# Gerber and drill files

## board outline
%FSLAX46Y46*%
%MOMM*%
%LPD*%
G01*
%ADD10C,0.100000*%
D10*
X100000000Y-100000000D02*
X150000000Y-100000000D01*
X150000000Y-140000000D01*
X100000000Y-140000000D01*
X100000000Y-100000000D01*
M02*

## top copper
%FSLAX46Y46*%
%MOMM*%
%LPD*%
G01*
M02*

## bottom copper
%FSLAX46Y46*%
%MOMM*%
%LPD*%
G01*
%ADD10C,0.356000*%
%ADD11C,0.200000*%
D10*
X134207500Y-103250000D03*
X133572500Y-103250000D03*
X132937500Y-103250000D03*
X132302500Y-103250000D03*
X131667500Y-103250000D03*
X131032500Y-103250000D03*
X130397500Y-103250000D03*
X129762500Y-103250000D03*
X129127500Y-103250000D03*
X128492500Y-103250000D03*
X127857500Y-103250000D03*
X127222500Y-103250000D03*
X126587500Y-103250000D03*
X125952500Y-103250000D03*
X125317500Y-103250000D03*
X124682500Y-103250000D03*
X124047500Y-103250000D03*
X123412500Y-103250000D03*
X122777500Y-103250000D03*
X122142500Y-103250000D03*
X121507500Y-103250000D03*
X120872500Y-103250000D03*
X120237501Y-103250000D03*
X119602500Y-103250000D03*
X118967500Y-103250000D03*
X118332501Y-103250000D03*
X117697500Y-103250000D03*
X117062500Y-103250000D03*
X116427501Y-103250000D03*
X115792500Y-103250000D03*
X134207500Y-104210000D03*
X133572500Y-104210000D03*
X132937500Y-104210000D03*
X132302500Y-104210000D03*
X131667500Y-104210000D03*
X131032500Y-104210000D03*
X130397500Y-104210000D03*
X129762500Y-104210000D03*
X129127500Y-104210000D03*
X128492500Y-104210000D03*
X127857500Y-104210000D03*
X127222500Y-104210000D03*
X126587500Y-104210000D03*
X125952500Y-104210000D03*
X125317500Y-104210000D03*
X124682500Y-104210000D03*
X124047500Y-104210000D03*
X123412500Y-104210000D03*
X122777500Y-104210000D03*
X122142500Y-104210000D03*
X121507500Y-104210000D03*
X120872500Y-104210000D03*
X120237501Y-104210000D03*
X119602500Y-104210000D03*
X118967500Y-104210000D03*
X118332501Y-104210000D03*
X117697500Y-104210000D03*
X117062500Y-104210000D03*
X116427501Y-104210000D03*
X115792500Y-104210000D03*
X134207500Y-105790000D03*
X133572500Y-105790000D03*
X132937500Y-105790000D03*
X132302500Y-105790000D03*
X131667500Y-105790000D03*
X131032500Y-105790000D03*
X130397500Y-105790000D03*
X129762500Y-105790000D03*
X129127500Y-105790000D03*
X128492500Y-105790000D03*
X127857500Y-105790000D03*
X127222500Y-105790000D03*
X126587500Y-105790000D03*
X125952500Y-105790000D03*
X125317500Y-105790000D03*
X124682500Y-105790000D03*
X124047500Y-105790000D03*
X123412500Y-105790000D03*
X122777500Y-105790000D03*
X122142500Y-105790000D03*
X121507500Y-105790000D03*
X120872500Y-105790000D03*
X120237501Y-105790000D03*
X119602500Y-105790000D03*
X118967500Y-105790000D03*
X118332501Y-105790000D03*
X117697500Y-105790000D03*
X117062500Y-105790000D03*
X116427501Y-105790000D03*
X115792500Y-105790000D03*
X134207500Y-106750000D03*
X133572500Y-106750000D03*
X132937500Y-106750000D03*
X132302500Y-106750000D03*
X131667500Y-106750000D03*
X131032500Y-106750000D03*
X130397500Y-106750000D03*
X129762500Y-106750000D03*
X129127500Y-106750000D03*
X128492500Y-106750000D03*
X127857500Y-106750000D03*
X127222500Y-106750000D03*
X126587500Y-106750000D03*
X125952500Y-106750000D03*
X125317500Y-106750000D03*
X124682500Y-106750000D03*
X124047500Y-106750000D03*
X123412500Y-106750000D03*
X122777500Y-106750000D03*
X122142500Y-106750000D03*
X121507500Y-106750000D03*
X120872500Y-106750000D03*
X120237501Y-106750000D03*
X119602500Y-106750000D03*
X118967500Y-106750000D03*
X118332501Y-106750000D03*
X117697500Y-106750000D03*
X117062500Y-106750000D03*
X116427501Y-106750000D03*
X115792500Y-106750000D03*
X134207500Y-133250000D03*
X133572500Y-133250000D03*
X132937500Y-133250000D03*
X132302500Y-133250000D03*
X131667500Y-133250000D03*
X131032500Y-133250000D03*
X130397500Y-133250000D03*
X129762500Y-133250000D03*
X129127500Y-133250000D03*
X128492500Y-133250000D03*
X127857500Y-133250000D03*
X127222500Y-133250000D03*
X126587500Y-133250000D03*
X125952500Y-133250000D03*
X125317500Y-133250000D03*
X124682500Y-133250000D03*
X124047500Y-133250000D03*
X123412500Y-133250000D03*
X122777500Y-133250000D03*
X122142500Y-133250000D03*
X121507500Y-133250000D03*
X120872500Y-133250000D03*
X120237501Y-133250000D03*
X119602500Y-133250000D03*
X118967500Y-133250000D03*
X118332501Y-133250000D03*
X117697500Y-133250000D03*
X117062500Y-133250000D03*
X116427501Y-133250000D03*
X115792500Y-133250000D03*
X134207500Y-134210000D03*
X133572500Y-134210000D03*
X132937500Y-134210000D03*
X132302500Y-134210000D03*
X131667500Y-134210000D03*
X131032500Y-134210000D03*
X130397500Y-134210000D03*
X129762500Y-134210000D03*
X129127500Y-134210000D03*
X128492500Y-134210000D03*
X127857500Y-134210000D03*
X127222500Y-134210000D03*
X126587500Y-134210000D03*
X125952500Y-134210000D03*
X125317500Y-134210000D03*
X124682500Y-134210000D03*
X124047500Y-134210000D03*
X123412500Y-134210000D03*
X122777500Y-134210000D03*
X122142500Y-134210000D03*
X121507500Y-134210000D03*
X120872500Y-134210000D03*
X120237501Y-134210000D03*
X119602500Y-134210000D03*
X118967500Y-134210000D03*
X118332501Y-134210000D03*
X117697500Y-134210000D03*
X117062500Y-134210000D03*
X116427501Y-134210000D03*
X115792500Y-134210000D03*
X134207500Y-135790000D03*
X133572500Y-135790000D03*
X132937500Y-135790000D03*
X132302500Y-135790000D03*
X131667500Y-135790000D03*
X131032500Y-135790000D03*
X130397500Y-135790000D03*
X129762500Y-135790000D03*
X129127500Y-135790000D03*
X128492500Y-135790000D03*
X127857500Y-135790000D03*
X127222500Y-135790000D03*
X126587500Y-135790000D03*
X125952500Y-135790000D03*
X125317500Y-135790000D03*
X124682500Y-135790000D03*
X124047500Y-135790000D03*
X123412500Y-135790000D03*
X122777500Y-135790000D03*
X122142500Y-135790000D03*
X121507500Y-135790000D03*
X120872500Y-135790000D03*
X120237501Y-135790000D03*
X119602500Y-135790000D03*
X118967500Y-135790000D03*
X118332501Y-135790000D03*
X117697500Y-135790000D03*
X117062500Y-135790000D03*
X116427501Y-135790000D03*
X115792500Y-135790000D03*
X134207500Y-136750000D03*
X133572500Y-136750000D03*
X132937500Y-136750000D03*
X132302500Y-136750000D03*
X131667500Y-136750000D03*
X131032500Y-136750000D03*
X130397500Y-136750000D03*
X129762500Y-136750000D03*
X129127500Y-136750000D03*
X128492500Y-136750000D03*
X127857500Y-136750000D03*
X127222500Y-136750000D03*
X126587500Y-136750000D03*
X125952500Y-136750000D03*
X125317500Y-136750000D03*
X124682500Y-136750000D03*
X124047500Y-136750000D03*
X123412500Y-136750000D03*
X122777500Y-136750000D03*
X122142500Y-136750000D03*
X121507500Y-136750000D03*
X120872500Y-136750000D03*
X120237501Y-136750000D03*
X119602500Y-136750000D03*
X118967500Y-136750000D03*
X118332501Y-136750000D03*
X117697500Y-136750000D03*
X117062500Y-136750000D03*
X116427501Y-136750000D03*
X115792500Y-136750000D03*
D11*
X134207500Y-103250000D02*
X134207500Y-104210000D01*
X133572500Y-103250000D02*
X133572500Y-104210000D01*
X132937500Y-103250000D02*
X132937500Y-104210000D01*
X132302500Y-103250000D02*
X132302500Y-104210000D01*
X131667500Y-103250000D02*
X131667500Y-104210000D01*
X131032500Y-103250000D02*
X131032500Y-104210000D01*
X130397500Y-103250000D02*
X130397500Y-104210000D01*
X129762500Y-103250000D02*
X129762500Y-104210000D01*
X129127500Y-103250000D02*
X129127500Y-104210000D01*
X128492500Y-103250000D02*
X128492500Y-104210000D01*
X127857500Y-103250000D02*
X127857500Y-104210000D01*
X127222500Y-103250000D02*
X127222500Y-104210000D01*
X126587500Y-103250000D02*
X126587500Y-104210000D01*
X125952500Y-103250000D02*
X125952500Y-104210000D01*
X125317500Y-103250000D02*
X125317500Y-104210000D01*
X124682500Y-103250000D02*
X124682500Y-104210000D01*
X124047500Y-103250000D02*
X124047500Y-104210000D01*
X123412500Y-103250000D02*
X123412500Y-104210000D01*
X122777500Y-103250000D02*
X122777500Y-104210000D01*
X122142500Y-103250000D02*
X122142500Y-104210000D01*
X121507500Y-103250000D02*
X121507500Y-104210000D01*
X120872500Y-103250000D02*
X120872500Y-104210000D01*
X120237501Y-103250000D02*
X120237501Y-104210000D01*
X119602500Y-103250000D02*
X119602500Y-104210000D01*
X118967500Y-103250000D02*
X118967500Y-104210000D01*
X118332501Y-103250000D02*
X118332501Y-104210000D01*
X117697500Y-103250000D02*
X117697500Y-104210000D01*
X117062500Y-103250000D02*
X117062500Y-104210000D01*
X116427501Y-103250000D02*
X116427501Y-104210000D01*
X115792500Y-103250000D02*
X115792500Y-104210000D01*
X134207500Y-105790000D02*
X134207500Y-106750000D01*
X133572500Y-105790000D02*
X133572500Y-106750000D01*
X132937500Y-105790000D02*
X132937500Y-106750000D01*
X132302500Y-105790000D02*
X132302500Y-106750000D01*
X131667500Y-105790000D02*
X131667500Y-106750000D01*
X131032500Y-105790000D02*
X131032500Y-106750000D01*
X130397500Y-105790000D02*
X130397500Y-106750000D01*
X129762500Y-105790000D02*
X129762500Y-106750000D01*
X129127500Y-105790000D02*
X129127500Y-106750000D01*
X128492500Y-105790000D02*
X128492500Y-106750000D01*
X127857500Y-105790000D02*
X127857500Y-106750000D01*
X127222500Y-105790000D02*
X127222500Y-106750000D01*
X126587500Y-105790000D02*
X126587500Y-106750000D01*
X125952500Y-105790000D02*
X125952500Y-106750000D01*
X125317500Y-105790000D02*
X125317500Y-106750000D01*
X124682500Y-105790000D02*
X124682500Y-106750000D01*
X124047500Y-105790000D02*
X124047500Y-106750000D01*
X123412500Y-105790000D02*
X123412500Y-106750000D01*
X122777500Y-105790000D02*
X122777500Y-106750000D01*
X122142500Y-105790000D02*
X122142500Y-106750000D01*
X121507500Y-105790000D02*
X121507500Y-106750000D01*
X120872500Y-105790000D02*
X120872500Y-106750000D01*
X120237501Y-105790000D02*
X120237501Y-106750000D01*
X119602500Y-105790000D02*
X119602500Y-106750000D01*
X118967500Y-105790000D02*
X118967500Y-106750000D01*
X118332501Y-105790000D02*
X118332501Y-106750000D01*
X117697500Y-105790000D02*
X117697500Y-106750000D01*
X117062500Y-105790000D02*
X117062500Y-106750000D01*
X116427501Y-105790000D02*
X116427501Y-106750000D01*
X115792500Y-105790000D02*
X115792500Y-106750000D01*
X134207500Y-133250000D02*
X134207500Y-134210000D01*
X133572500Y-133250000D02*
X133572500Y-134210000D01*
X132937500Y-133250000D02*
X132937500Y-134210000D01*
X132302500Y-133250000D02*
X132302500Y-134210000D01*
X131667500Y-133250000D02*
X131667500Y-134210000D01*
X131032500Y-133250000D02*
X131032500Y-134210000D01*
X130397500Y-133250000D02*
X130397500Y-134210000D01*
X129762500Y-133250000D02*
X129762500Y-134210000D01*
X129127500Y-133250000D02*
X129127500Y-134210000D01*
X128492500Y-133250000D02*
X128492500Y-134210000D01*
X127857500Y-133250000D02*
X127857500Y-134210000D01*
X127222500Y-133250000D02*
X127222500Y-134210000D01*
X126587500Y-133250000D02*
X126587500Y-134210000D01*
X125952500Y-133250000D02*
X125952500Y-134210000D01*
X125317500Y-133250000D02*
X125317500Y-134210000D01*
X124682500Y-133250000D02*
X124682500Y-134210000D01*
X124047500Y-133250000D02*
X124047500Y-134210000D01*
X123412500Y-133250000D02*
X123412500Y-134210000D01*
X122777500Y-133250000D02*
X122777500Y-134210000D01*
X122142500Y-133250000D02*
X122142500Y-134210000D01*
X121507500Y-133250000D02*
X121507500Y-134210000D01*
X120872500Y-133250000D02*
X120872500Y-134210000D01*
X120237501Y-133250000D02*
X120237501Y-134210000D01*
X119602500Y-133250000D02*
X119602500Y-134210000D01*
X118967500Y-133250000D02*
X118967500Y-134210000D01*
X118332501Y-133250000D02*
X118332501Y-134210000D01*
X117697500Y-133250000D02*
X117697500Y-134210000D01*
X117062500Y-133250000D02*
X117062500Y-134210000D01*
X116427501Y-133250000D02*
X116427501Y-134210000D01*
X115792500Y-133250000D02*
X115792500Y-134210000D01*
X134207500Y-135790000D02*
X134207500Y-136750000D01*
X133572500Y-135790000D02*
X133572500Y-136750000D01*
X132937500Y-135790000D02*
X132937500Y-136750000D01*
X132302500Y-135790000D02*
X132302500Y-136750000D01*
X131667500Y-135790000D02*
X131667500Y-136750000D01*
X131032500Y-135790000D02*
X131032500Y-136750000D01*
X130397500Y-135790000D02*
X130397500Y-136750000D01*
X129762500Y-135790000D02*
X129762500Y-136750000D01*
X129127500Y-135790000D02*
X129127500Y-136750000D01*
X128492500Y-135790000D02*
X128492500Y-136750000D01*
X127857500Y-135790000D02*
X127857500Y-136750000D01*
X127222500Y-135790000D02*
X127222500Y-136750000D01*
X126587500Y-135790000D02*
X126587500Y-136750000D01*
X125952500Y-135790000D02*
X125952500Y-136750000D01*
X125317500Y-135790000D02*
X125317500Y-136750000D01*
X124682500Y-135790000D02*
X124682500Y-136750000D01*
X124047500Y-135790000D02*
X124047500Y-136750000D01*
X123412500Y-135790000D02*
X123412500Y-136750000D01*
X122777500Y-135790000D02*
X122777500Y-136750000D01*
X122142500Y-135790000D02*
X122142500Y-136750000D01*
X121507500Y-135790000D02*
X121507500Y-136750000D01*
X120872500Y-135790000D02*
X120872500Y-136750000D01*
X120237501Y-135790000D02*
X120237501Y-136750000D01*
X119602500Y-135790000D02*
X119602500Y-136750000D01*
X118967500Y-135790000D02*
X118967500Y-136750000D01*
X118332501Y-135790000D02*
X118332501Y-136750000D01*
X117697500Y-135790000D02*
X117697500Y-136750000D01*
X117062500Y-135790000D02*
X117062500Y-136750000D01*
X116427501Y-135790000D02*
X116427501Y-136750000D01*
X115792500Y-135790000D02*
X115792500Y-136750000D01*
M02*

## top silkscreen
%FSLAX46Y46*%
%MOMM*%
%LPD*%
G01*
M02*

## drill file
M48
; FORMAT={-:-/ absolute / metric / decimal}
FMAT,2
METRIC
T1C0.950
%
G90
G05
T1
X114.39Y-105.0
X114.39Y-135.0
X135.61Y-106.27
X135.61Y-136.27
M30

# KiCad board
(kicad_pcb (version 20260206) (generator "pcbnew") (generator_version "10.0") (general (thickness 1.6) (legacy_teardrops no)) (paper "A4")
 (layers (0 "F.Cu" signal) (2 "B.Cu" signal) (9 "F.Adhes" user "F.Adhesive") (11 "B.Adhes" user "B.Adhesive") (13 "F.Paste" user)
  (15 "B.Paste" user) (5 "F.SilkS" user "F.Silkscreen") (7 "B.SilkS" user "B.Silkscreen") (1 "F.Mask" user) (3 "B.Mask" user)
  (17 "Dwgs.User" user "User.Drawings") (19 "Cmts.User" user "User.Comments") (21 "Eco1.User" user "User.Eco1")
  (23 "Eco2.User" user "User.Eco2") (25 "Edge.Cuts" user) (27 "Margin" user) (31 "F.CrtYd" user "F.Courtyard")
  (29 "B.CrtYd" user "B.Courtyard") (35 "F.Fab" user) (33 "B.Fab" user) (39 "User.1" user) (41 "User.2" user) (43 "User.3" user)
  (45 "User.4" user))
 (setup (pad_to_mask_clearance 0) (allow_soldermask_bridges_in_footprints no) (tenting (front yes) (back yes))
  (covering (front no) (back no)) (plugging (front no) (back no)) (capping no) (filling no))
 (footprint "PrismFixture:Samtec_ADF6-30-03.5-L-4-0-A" (layer "B.Cu") (at 125 105)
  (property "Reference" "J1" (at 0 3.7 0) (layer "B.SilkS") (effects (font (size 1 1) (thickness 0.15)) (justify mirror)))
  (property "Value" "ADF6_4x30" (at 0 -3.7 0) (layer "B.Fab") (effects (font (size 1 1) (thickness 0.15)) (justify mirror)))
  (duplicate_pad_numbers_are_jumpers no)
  (pad "" np_thru_hole circle (at -10.61 0) (size 0.95 0.95) (drill 0.95) (layers "*.Cu" "*.Mask"))
  (pad "" np_thru_hole circle (at 10.61 1.27) (size 0.95 0.95) (drill 0.95) (layers "*.Cu" "*.Mask"))
  (pad "A01" smd circle (at 9.2075 -1.75) (size 0.356 0.356) (layers "B.Cu" "B.Mask" "B.Paste") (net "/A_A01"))
  (pad "A02" smd circle (at 8.5725 -1.75) (size 0.356 0.356) (layers "B.Cu" "B.Mask" "B.Paste") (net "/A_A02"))
  (pad "A03" smd circle (at 7.9375 -1.75) (size 0.356 0.356) (layers "B.Cu" "B.Mask" "B.Paste") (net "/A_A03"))
  (pad "A04" smd circle (at 7.3025 -1.75) (size 0.356 0.356) (layers "B.Cu" "B.Mask" "B.Paste") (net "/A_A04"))
  (pad "A05" smd circle (at 6.6675 -1.75) (size 0.356 0.356) (layers "B.Cu" "B.Mask" "B.Paste") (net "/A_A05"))
  (pad "A06" smd circle (at 6.0325 -1.75) (size 0.356 0.356) (layers "B.Cu" "B.Mask" "B.Paste") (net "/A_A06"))
  (pad "A07" smd circle (at 5.3975 -1.75) (size 0.356 0.356) (layers "B.Cu" "B.Mask" "B.Paste") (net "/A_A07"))
  (pad "A08" smd circle (at 4.7625 -1.75) (size 0.356 0.356) (layers "B.Cu" "B.Mask" "B.Paste") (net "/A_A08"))
  (pad "A09" smd circle (at 4.1275 -1.75) (size 0.356 0.356) (layers "B.Cu" "B.Mask" "B.Paste") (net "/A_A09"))
  (pad "A10" smd circle (at 3.4925 -1.75) (size 0.356 0.356) (layers "B.Cu" "B.Mask" "B.Paste") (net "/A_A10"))
  (pad "A11" smd circle (at 2.8575 -1.75) (size 0.356 0.356) (layers "B.Cu" "B.Mask" "B.Paste") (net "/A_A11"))
  (pad "A12" smd circle (at 2.2225 -1.75) (size 0.356 0.356) (layers "B.Cu" "B.Mask" "B.Paste") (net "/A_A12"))
  (pad "A13" smd circle (at 1.5875 -1.75) (size 0.356 0.356) (layers "B.Cu" "B.Mask" "B.Paste") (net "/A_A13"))
  (pad "A14" smd circle (at 0.9525 -1.75) (size 0.356 0.356) (layers "B.Cu" "B.Mask" "B.Paste") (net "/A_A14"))
  (pad "A15" smd circle (at 0.3175 -1.75) (size 0.356 0.356) (layers "B.Cu" "B.Mask" "B.Paste") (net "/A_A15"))
  (pad "A16" smd circle (at -0.3175 -1.75) (size 0.356 0.356) (layers "B.Cu" "B.Mask" "B.Paste") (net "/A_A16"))
  (pad "A17" smd circle (at -0.9525 -1.75) (size 0.356 0.356) (layers "B.Cu" "B.Mask" "B.Paste") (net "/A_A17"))
  (pad "A18" smd circle (at -1.5875 -1.75) (size 0.356 0.356) (layers "B.Cu" "B.Mask" "B.Paste") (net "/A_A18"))
  (pad "A19" smd circle (at -2.2225 -1.75) (size 0.356 0.356) (layers "B.Cu" "B.Mask" "B.Paste") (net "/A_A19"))
  (pad "A20" smd circle (at -2.8575 -1.75) (size 0.356 0.356) (layers "B.Cu" "B.Mask" "B.Paste") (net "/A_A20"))
  (pad "A21" smd circle (at -3.4925 -1.75) (size 0.356 0.356) (layers "B.Cu" "B.Mask" "B.Paste") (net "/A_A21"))
  (pad "A22" smd circle (at -4.1275 -1.75) (size 0.356 0.356) (layers "B.Cu" "B.Mask" "B.Paste") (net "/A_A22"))
  (pad "A23" smd circle (at -4.762499 -1.75) (size 0.356 0.356) (layers "B.Cu" "B.Mask" "B.Paste") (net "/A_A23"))
  (pad "A24" smd circle (at -5.3975 -1.75) (size 0.356 0.356) (layers "B.Cu" "B.Mask" "B.Paste") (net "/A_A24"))
  (pad "A25" smd circle (at -6.0325 -1.75) (size 0.356 0.356) (layers "B.Cu" "B.Mask" "B.Paste") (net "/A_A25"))
  (pad "A26" smd circle (at -6.667499 -1.75) (size 0.356 0.356) (layers "B.Cu" "B.Mask" "B.Paste") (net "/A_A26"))
  (pad "A27" smd circle (at -7.3025 -1.75) (size 0.356 0.356) (layers "B.Cu" "B.Mask" "B.Paste") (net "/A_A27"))
  (pad "A28" smd circle (at -7.9375 -1.75) (size 0.356 0.356) (layers "B.Cu" "B.Mask" "B.Paste") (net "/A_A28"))
  (pad "A29" smd circle (at -8.572499 -1.75) (size 0.356 0.356) (layers "B.Cu" "B.Mask" "B.Paste") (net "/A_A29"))
  (pad "A30" smd circle (at -9.2075 -1.75) (size 0.356 0.356) (layers "B.Cu" "B.Mask" "B.Paste") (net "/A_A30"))
  (pad "B01" smd circle (at 9.2075 -0.79) (size 0.356 0.356) (layers "B.Cu" "B.Mask" "B.Paste") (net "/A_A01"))
  (pad "B02" smd circle (at 8.5725 -0.79) (size 0.356 0.356) (layers "B.Cu" "B.Mask" "B.Paste") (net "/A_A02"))
  (pad "B03" smd circle (at 7.9375 -0.79) (size 0.356 0.356) (layers "B.Cu" "B.Mask" "B.Paste") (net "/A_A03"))
  (pad "B04" smd circle (at 7.3025 -0.79) (size 0.356 0.356) (layers "B.Cu" "B.Mask" "B.Paste") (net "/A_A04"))
  (pad "B05" smd circle (at 6.6675 -0.79) (size 0.356 0.356) (layers "B.Cu" "B.Mask" "B.Paste") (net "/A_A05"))
  (pad "B06" smd circle (at 6.0325 -0.79) (size 0.356 0.356) (layers "B.Cu" "B.Mask" "B.Paste") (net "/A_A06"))
  (pad "B07" smd circle (at 5.3975 -0.79) (size 0.356 0.356) (layers "B.Cu" "B.Mask" "B.Paste") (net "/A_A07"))
  (pad "B08" smd circle (at 4.7625 -0.79) (size 0.356 0.356) (layers "B.Cu" "B.Mask" "B.Paste") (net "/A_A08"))
  (pad "B09" smd circle (at 4.1275 -0.79) (size 0.356 0.356) (layers "B.Cu" "B.Mask" "B.Paste") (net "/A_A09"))
  (pad "B10" smd circle (at 3.4925 -0.79) (size 0.356 0.356) (layers "B.Cu" "B.Mask" "B.Paste") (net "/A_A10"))
  (pad "B11" smd circle (at 2.8575 -0.79) (size 0.356 0.356) (layers "B.Cu" "B.Mask" "B.Paste") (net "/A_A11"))
  (pad "B12" smd circle (at 2.2225 -0.79) (size 0.356 0.356) (layers "B.Cu" "B.Mask" "B.Paste") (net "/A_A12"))
  (pad "B13" smd circle (at 1.5875 -0.79) (size 0.356 0.356) (layers "B.Cu" "B.Mask" "B.Paste") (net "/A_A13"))
  (pad "B14" smd circle (at 0.9525 -0.79) (size 0.356 0.356) (layers "B.Cu" "B.Mask" "B.Paste") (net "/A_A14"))
  (pad "B15" smd circle (at 0.3175 -0.79) (size 0.356 0.356) (layers "B.Cu" "B.Mask" "B.Paste") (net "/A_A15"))
  (pad "B16" smd circle (at -0.3175 -0.79) (size 0.356 0.356) (layers "B.Cu" "B.Mask" "B.Paste") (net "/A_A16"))
  (pad "B17" smd circle (at -0.9525 -0.79) (size 0.356 0.356) (layers "B.Cu" "B.Mask" "B.Paste") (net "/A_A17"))
  (pad "B18" smd circle (at -1.5875 -0.79) (size 0.356 0.356) (layers "B.Cu" "B.Mask" "B.Paste") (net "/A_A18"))
  (pad "B19" smd circle (at -2.2225 -0.79) (size 0.356 0.356) (layers "B.Cu" "B.Mask" "B.Paste") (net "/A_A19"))
  (pad "B20" smd circle (at -2.8575 -0.79) (size 0.356 0.356) (layers "B.Cu" "B.Mask" "B.Paste") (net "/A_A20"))
  (pad "B21" smd circle (at -3.4925 -0.79) (size 0.356 0.356) (layers "B.Cu" "B.Mask" "B.Paste") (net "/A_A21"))
  (pad "B22" smd circle (at -4.1275 -0.79) (size 0.356 0.356) (layers "B.Cu" "B.Mask" "B.Paste") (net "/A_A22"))
  (pad "B23" smd circle (at -4.762499 -0.79) (size 0.356 0.356) (layers "B.Cu" "B.Mask" "B.Paste") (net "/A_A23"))
  (pad "B24" smd circle (at -5.3975 -0.79) (size 0.356 0.356) (layers "B.Cu" "B.Mask" "B.Paste") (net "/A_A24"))
  (pad "B25" smd circle (at -6.0325 -0.79) (size 0.356 0.356) (layers "B.Cu" "B.Mask" "B.Paste") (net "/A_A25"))
  (pad "B26" smd circle (at -6.667499 -0.79) (size 0.356 0.356) (layers "B.Cu" "B.Mask" "B.Paste") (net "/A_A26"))
  (pad "B27" smd circle (at -7.3025 -0.79) (size 0.356 0.356) (layers "B.Cu" "B.Mask" "B.Paste") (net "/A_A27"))
  (pad "B28" smd circle (at -7.9375 -0.79) (size 0.356 0.356) (layers "B.Cu" "B.Mask" "B.Paste") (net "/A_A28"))
  (pad "B29" smd circle (at -8.572499 -0.79) (size 0.356 0.356) (layers "B.Cu" "B.Mask" "B.Paste") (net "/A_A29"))
  (pad "B30" smd circle (at -9.2075 -0.79) (size 0.356 0.356) (layers "B.Cu" "B.Mask" "B.Paste") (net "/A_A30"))
  (pad "C01" smd circle (at 9.2075 0.79) (size 0.356 0.356) (layers "B.Cu" "B.Mask" "B.Paste") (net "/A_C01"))
  (pad "C02" smd circle (at 8.5725 0.79) (size 0.356 0.356) (layers "B.Cu" "B.Mask" "B.Paste") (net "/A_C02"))
  (pad "C03" smd circle (at 7.9375 0.79) (size 0.356 0.356) (layers "B.Cu" "B.Mask" "B.Paste") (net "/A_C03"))
  (pad "C04" smd circle (at 7.3025 0.79) (size 0.356 0.356) (layers "B.Cu" "B.Mask" "B.Paste") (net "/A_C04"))
  (pad "C05" smd circle (at 6.6675 0.79) (size 0.356 0.356) (layers "B.Cu" "B.Mask" "B.Paste") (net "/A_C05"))
  (pad "C06" smd circle (at 6.0325 0.79) (size 0.356 0.356) (layers "B.Cu" "B.Mask" "B.Paste") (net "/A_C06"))
  (pad "C07" smd circle (at 5.3975 0.79) (size 0.356 0.356) (layers "B.Cu" "B.Mask" "B.Paste") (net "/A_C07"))
  (pad "C08" smd circle (at 4.7625 0.79) (size 0.356 0.356) (layers "B.Cu" "B.Mask" "B.Paste") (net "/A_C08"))
  (pad "C09" smd circle (at 4.1275 0.79) (size 0.356 0.356) (layers "B.Cu" "B.Mask" "B.Paste") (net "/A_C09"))
  (pad "C10" smd circle (at 3.4925 0.79) (size 0.356 0.356) (layers "B.Cu" "B.Mask" "B.Paste") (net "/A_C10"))
  (pad "C11" smd circle (at 2.8575 0.79) (size 0.356 0.356) (layers "B.Cu" "B.Mask" "B.Paste") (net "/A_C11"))
  (pad "C12" smd circle (at 2.2225 0.79) (size 0.356 0.356) (layers "B.Cu" "B.Mask" "B.Paste") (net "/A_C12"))
  (pad "C13" smd circle (at 1.5875 0.79) (size 0.356 0.356) (layers "B.Cu" "B.Mask" "B.Paste") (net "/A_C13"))
  (pad "C14" smd circle (at 0.9525 0.79) (size 0.356 0.356) (layers "B.Cu" "B.Mask" "B.Paste") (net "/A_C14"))
  (pad "C15" smd circle (at 0.3175 0.79) (size 0.356 0.356) (layers "B.Cu" "B.Mask" "B.Paste") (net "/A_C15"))
  (pad "C16" smd circle (at -0.3175 0.79) (size 0.356 0.356) (layers "B.Cu" "B.Mask" "B.Paste") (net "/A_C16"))
  (pad "C17" smd circle (at -0.9525 0.79) (size 0.356 0.356) (layers "B.Cu" "B.Mask" "B.Paste") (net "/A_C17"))
  (pad "C18" smd circle (at -1.5875 0.79) (size 0.356 0.356) (layers "B.Cu" "B.Mask" "B.Paste") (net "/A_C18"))
  (pad "C19" smd circle (at -2.2225 0.79) (size 0.356 0.356) (layers "B.Cu" "B.Mask" "B.Paste") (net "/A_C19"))
  (pad "C20" smd circle (at -2.8575 0.79) (size 0.356 0.356) (layers "B.Cu" "B.Mask" "B.Paste") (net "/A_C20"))
  (pad "C21" smd circle (at -3.4925 0.79) (size 0.356 0.356) (layers "B.Cu" "B.Mask" "B.Paste") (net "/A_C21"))
  (pad "C22" smd circle (at -4.1275 0.79) (size 0.356 0.356) (layers "B.Cu" "B.Mask" "B.Paste") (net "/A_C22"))
  (pad "C23" smd circle (at -4.762499 0.79) (size 0.356 0.356) (layers "B.Cu" "B.Mask" "B.Paste") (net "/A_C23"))
  (pad "C24" smd circle (at -5.3975 0.79) (size 0.356 0.356) (layers "B.Cu" "B.Mask" "B.Paste") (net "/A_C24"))
  (pad "C25" smd circle (at -6.0325 0.79) (size 0.356 0.356) (layers "B.Cu" "B.Mask" "B.Paste") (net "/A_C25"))
  (pad "C26" smd circle (at -6.667499 0.79) (size 0.356 0.356) (layers "B.Cu" "B.Mask" "B.Paste") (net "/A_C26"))
  (pad "C27" smd circle (at -7.3025 0.79) (size 0.356 0.356) (layers "B.Cu" "B.Mask" "B.Paste") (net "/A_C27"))
  (pad "C28" smd circle (at -7.9375 0.79) (size 0.356 0.356) (layers "B.Cu" "B.Mask" "B.Paste") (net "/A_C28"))
  (pad "C29" smd circle (at -8.572499 0.79) (size 0.356 0.356) (layers "B.Cu" "B.Mask" "B.Paste") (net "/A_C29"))
  (pad "C30" smd circle (at -9.2075 0.79) (size 0.356 0.356) (layers "B.Cu" "B.Mask" "B.Paste") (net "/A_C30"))
  (pad "D01" smd circle (at 9.2075 1.75) (size 0.356 0.356) (layers "B.Cu" "B.Mask" "B.Paste") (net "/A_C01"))
  (pad "D02" smd circle (at 8.5725 1.75) (size 0.356 0.356) (layers "B.Cu" "B.Mask" "B.Paste") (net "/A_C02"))
  (pad "D03" smd circle (at 7.9375 1.75) (size 0.356 0.356) (layers "B.Cu" "B.Mask" "B.Paste") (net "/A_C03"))
  (pad "D04" smd circle (at 7.3025 1.75) (size 0.356 0.356) (layers "B.Cu" "B.Mask" "B.Paste") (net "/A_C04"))
  (pad "D05" smd circle (at 6.6675 1.75) (size 0.356 0.356) (layers "B.Cu" "B.Mask" "B.Paste") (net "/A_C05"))
  (pad "D06" smd circle (at 6.0325 1.75) (size 0.356 0.356) (layers "B.Cu" "B.Mask" "B.Paste") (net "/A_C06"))
  (pad "D07" smd circle (at 5.3975 1.75) (size 0.356 0.356) (layers "B.Cu" "B.Mask" "B.Paste") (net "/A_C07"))
  (pad "D08" smd circle (at 4.7625 1.75) (size 0.356 0.356) (layers "B.Cu" "B.Mask" "B.Paste") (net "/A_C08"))
  (pad "D09" smd circle (at 4.1275 1.75) (size 0.356 0.356) (layers "B.Cu" "B.Mask" "B.Paste") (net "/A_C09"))
  (pad "D10" smd circle (at 3.4925 1.75) (size 0.356 0.356) (layers "B.Cu" "B.Mask" "B.Paste") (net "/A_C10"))
  (pad "D11" smd circle (at 2.8575 1.75) (size 0.356 0.356) (layers "B.Cu" "B.Mask" "B.Paste") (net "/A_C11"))
  (pad "D12" smd circle (at 2.2225 1.75) (size 0.356 0.356) (layers "B.Cu" "B.Mask" "B.Paste") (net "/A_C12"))
  (pad "D13" smd circle (at 1.5875 1.75) (size 0.356 0.356) (layers "B.Cu" "B.Mask" "B.Paste") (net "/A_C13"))
  (pad "D14" smd circle (at 0.9525 1.75) (size 0.356 0.356) (layers "B.Cu" "B.Mask" "B.Paste") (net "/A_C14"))
  (pad "D15" smd circle (at 0.3175 1.75) (size 0.356 0.356) (layers "B.Cu" "B.Mask" "B.Paste") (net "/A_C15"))
  (pad "D16" smd circle (at -0.3175 1.75) (size 0.356 0.356) (layers "B.Cu" "B.Mask" "B.Paste") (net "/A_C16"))
  (pad "D17" smd circle (at -0.9525 1.75) (size 0.356 0.356) (layers "B.Cu" "B.Mask" "B.Paste") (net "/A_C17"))
  (pad "D18" smd circle (at -1.5875 1.75) (size 0.356 0.356) (layers "B.Cu" "B.Mask" "B.Paste") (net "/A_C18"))
  (pad "D19" smd circle (at -2.2225 1.75) (size 0.356 0.356) (layers "B.Cu" "B.Mask" "B.Paste") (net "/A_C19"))
  (pad "D20" smd circle (at -2.8575 1.75) (size 0.356 0.356) (layers "B.Cu" "B.Mask" "B.Paste") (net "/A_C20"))
  (pad "D21" smd circle (at -3.4925 1.75) (size 0.356 0.356) (layers "B.Cu" "B.Mask" "B.Paste") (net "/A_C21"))
  (pad "D22" smd circle (at -4.1275 1.75) (size 0.356 0.356) (layers "B.Cu" "B.Mask" "B.Paste") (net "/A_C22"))
  (pad "D23" smd circle (at -4.762499 1.75) (size 0.356 0.356) (layers "B.Cu" "B.Mask" "B.Paste") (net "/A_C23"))
  (pad "D24" smd circle (at -5.3975 1.75) (size 0.356 0.356) (layers "B.Cu" "B.Mask" "B.Paste") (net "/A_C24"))
  (pad "D25" smd circle (at -6.0325 1.75) (size 0.356 0.356) (layers "B.Cu" "B.Mask" "B.Paste") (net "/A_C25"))
  (pad "D26" smd circle (at -6.667499 1.75) (size 0.356 0.356) (layers "B.Cu" "B.Mask" "B.Paste") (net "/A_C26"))
  (pad "D27" smd circle (at -7.3025 1.75) (size 0.356 0.356) (layers "B.Cu" "B.Mask" "B.Paste") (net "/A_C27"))
  (pad "D28" smd circle (at -7.9375 1.75) (size 0.356 0.356) (layers "B.Cu" "B.Mask" "B.Paste") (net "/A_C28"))
  (pad "D29" smd circle (at -8.572499 1.75) (size 0.356 0.356) (layers "B.Cu" "B.Mask" "B.Paste") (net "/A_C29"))
  (pad "D30" smd circle (at -9.2075 1.75) (size 0.356 0.356) (layers "B.Cu" "B.Mask" "B.Paste") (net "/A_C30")))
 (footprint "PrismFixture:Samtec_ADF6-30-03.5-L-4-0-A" (layer "B.Cu") (at 125 135)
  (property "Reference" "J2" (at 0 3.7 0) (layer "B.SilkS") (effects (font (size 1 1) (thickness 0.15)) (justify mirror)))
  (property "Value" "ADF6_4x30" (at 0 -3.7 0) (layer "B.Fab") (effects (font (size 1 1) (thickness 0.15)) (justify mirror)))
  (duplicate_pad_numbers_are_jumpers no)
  (pad "" np_thru_hole circle (at -10.61 0) (size 0.95 0.95) (drill 0.95) (layers "*.Cu" "*.Mask"))
  (pad "" np_thru_hole circle (at 10.61 1.27) (size 0.95 0.95) (drill 0.95) (layers "*.Cu" "*.Mask"))
  (pad "A01" smd circle (at 9.2075 -1.75) (size 0.356 0.356) (layers "B.Cu" "B.Mask" "B.Paste") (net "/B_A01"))
  (pad "A02" smd circle (at 8.5725 -1.75) (size 0.356 0.356) (layers "B.Cu" "B.Mask" "B.Paste") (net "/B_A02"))
  (pad "A03" smd circle (at 7.9375 -1.75) (size 0.356 0.356) (layers "B.Cu" "B.Mask" "B.Paste") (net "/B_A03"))
  (pad "A04" smd circle (at 7.3025 -1.75) (size 0.356 0.356) (layers "B.Cu" "B.Mask" "B.Paste") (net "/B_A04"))
  (pad "A05" smd circle (at 6.6675 -1.75) (size 0.356 0.356) (layers "B.Cu" "B.Mask" "B.Paste") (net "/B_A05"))
  (pad "A06" smd circle (at 6.0325 -1.75) (size 0.356 0.356) (layers "B.Cu" "B.Mask" "B.Paste") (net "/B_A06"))
  (pad "A07" smd circle (at 5.3975 -1.75) (size 0.356 0.356) (layers "B.Cu" "B.Mask" "B.Paste") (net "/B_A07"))
  (pad "A08" smd circle (at 4.7625 -1.75) (size 0.356 0.356) (layers "B.Cu" "B.Mask" "B.Paste") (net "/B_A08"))
  (pad "A09" smd circle (at 4.1275 -1.75) (size 0.356 0.356) (layers "B.Cu" "B.Mask" "B.Paste") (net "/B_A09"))
  (pad "A10" smd circle (at 3.4925 -1.75) (size 0.356 0.356) (layers "B.Cu" "B.Mask" "B.Paste") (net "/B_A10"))
  (pad "A11" smd circle (at 2.8575 -1.75) (size 0.356 0.356) (layers "B.Cu" "B.Mask" "B.Paste") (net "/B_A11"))
  (pad "A12" smd circle (at 2.2225 -1.75) (size 0.356 0.356) (layers "B.Cu" "B.Mask" "B.Paste") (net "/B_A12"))
  (pad "A13" smd circle (at 1.5875 -1.75) (size 0.356 0.356) (layers "B.Cu" "B.Mask" "B.Paste") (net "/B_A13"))
  (pad "A14" smd circle (at 0.9525 -1.75) (size 0.356 0.356) (layers "B.Cu" "B.Mask" "B.Paste") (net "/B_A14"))
  (pad "A15" smd circle (at 0.3175 -1.75) (size 0.356 0.356) (layers "B.Cu" "B.Mask" "B.Paste") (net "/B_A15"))
  (pad "A16" smd circle (at -0.3175 -1.75) (size 0.356 0.356) (layers "B.Cu" "B.Mask" "B.Paste") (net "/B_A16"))
  (pad "A17" smd circle (at -0.9525 -1.75) (size 0.356 0.356) (layers "B.Cu" "B.Mask" "B.Paste") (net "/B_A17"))
  (pad "A18" smd circle (at -1.5875 -1.75) (size 0.356 0.356) (layers "B.Cu" "B.Mask" "B.Paste") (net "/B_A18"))
  (pad "A19" smd circle (at -2.2225 -1.75) (size 0.356 0.356) (layers "B.Cu" "B.Mask" "B.Paste") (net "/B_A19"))
  (pad "A20" smd circle (at -2.8575 -1.75) (size 0.356 0.356) (layers "B.Cu" "B.Mask" "B.Paste") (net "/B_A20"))
  (pad "A21" smd circle (at -3.4925 -1.75) (size 0.356 0.356) (layers "B.Cu" "B.Mask" "B.Paste") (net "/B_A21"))
  (pad "A22" smd circle (at -4.1275 -1.75) (size 0.356 0.356) (layers "B.Cu" "B.Mask" "B.Paste") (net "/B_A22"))
  (pad "A23" smd circle (at -4.762499 -1.75) (size 0.356 0.356) (layers "B.Cu" "B.Mask" "B.Paste") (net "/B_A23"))
  (pad "A24" smd circle (at -5.3975 -1.75) (size 0.356 0.356) (layers "B.Cu" "B.Mask" "B.Paste") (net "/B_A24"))
  (pad "A25" smd circle (at -6.0325 -1.75) (size 0.356 0.356) (layers "B.Cu" "B.Mask" "B.Paste") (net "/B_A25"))
  (pad "A26" smd circle (at -6.667499 -1.75) (size 0.356 0.356) (layers "B.Cu" "B.Mask" "B.Paste") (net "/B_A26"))
  (pad "A27" smd circle (at -7.3025 -1.75) (size 0.356 0.356) (layers "B.Cu" "B.Mask" "B.Paste") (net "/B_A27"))
  (pad "A28" smd circle (at -7.9375 -1.75) (size 0.356 0.356) (layers "B.Cu" "B.Mask" "B.Paste") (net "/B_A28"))
  (pad "A29" smd circle (at -8.572499 -1.75) (size 0.356 0.356) (layers "B.Cu" "B.Mask" "B.Paste") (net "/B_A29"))
  (pad "A30" smd circle (at -9.2075 -1.75) (size 0.356 0.356) (layers "B.Cu" "B.Mask" "B.Paste") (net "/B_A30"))
  (pad "B01" smd circle (at 9.2075 -0.79) (size 0.356 0.356) (layers "B.Cu" "B.Mask" "B.Paste") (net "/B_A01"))
  (pad "B02" smd circle (at 8.5725 -0.79) (size 0.356 0.356) (layers "B.Cu" "B.Mask" "B.Paste") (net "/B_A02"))
  (pad "B03" smd circle (at 7.9375 -0.79) (size 0.356 0.356) (layers "B.Cu" "B.Mask" "B.Paste") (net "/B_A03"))
  (pad "B04" smd circle (at 7.3025 -0.79) (size 0.356 0.356) (layers "B.Cu" "B.Mask" "B.Paste") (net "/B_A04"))
  (pad "B05" smd circle (at 6.6675 -0.79) (size 0.356 0.356) (layers "B.Cu" "B.Mask" "B.Paste") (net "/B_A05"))
  (pad "B06" smd circle (at 6.0325 -0.79) (size 0.356 0.356) (layers "B.Cu" "B.Mask" "B.Paste") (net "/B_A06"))
  (pad "B07" smd circle (at 5.3975 -0.79) (size 0.356 0.356) (layers "B.Cu" "B.Mask" "B.Paste") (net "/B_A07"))
  (pad "B08" smd circle (at 4.7625 -0.79) (size 0.356 0.356) (layers "B.Cu" "B.Mask" "B.Paste") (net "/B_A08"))
  (pad "B09" smd circle (at 4.1275 -0.79) (size 0.356 0.356) (layers "B.Cu" "B.Mask" "B.Paste") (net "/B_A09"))
  (pad "B10" smd circle (at 3.4925 -0.79) (size 0.356 0.356) (layers "B.Cu" "B.Mask" "B.Paste") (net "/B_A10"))
  (pad "B11" smd circle (at 2.8575 -0.79) (size 0.356 0.356) (layers "B.Cu" "B.Mask" "B.Paste") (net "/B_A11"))
  (pad "B12" smd circle (at 2.2225 -0.79) (size 0.356 0.356) (layers "B.Cu" "B.Mask" "B.Paste") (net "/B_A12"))
  (pad "B13" smd circle (at 1.5875 -0.79) (size 0.356 0.356) (layers "B.Cu" "B.Mask" "B.Paste") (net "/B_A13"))
  (pad "B14" smd circle (at 0.9525 -0.79) (size 0.356 0.356) (layers "B.Cu" "B.Mask" "B.Paste") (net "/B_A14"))
  (pad "B15" smd circle (at 0.3175 -0.79) (size 0.356 0.356) (layers "B.Cu" "B.Mask" "B.Paste") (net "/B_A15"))
  (pad "B16" smd circle (at -0.3175 -0.79) (size 0.356 0.356) (layers "B.Cu" "B.Mask" "B.Paste") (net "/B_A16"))
  (pad "B17" smd circle (at -0.9525 -0.79) (size 0.356 0.356) (layers "B.Cu" "B.Mask" "B.Paste") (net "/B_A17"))
  (pad "B18" smd circle (at -1.5875 -0.79) (size 0.356 0.356) (layers "B.Cu" "B.Mask" "B.Paste") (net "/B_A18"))
  (pad "B19" smd circle (at -2.2225 -0.79) (size 0.356 0.356) (layers "B.Cu" "B.Mask" "B.Paste") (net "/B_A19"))
  (pad "B20" smd circle (at -2.8575 -0.79) (size 0.356 0.356) (layers "B.Cu" "B.Mask" "B.Paste") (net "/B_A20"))
  (pad "B21" smd circle (at -3.4925 -0.79) (size 0.356 0.356) (layers "B.Cu" "B.Mask" "B.Paste") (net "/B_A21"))
  (pad "B22" smd circle (at -4.1275 -0.79) (size 0.356 0.356) (layers "B.Cu" "B.Mask" "B.Paste") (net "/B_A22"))
  (pad "B23" smd circle (at -4.762499 -0.79) (size 0.356 0.356) (layers "B.Cu" "B.Mask" "B.Paste") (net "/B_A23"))
  (pad "B24" smd circle (at -5.3975 -0.79) (size 0.356 0.356) (layers "B.Cu" "B.Mask" "B.Paste") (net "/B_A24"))
  (pad "B25" smd circle (at -6.0325 -0.79) (size 0.356 0.356) (layers "B.Cu" "B.Mask" "B.Paste") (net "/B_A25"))
  (pad "B26" smd circle (at -6.667499 -0.79) (size 0.356 0.356) (layers "B.Cu" "B.Mask" "B.Paste") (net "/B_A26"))
  (pad "B27" smd circle (at -7.3025 -0.79) (size 0.356 0.356) (layers "B.Cu" "B.Mask" "B.Paste") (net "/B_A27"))
  (pad "B28" smd circle (at -7.9375 -0.79) (size 0.356 0.356) (layers "B.Cu" "B.Mask" "B.Paste") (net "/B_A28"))
  (pad "B29" smd circle (at -8.572499 -0.79) (size 0.356 0.356) (layers "B.Cu" "B.Mask" "B.Paste") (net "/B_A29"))
  (pad "B30" smd circle (at -9.2075 -0.79) (size 0.356 0.356) (layers "B.Cu" "B.Mask" "B.Paste") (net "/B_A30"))
  (pad "C01" smd circle (at 9.2075 0.79) (size 0.356 0.356) (layers "B.Cu" "B.Mask" "B.Paste") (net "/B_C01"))
  (pad "C02" smd circle (at 8.5725 0.79) (size 0.356 0.356) (layers "B.Cu" "B.Mask" "B.Paste") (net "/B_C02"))
  (pad "C03" smd circle (at 7.9375 0.79) (size 0.356 0.356) (layers "B.Cu" "B.Mask" "B.Paste") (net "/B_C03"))
  (pad "C04" smd circle (at 7.3025 0.79) (size 0.356 0.356) (layers "B.Cu" "B.Mask" "B.Paste") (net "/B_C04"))
  (pad "C05" smd circle (at 6.6675 0.79) (size 0.356 0.356) (layers "B.Cu" "B.Mask" "B.Paste") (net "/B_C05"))
  (pad "C06" smd circle (at 6.0325 0.79) (size 0.356 0.356) (layers "B.Cu" "B.Mask" "B.Paste") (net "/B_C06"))
  (pad "C07" smd circle (at 5.3975 0.79) (size 0.356 0.356) (layers "B.Cu" "B.Mask" "B.Paste") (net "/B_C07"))
  (pad "C08" smd circle (at 4.7625 0.79) (size 0.356 0.356) (layers "B.Cu" "B.Mask" "B.Paste") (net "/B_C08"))
  (pad "C09" smd circle (at 4.1275 0.79) (size 0.356 0.356) (layers "B.Cu" "B.Mask" "B.Paste") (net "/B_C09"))
  (pad "C10" smd circle (at 3.4925 0.79) (size 0.356 0.356) (layers "B.Cu" "B.Mask" "B.Paste") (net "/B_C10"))
  (pad "C11" smd circle (at 2.8575 0.79) (size 0.356 0.356) (layers "B.Cu" "B.Mask" "B.Paste") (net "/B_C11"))
  (pad "C12" smd circle (at 2.2225 0.79) (size 0.356 0.356) (layers "B.Cu" "B.Mask" "B.Paste") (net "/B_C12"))
  (pad "C13" smd circle (at 1.5875 0.79) (size 0.356 0.356) (layers "B.Cu" "B.Mask" "B.Paste") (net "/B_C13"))
  (pad "C14" smd circle (at 0.9525 0.79) (size 0.356 0.356) (layers "B.Cu" "B.Mask" "B.Paste") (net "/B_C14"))
  (pad "C15" smd circle (at 0.3175 0.79) (size 0.356 0.356) (layers "B.Cu" "B.Mask" "B.Paste") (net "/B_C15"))
  (pad "C16" smd circle (at -0.3175 0.79) (size 0.356 0.356) (layers "B.Cu" "B.Mask" "B.Paste") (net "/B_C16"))
  (pad "C17" smd circle (at -0.9525 0.79) (size 0.356 0.356) (layers "B.Cu" "B.Mask" "B.Paste") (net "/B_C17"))
  (pad "C18" smd circle (at -1.5875 0.79) (size 0.356 0.356) (layers "B.Cu" "B.Mask" "B.Paste") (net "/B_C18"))
  (pad "C19" smd circle (at -2.2225 0.79) (size 0.356 0.356) (layers "B.Cu" "B.Mask" "B.Paste") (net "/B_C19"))
  (pad "C20" smd circle (at -2.8575 0.79) (size 0.356 0.356) (layers "B.Cu" "B.Mask" "B.Paste") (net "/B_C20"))
  (pad "C21" smd circle (at -3.4925 0.79) (size 0.356 0.356) (layers "B.Cu" "B.Mask" "B.Paste") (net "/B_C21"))
  (pad "C22" smd circle (at -4.1275 0.79) (size 0.356 0.356) (layers "B.Cu" "B.Mask" "B.Paste") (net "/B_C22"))
  (pad "C23" smd circle (at -4.762499 0.79) (size 0.356 0.356) (layers "B.Cu" "B.Mask" "B.Paste") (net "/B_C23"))
  (pad "C24" smd circle (at -5.3975 0.79) (size 0.356 0.356) (layers "B.Cu" "B.Mask" "B.Paste") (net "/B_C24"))
  (pad "C25" smd circle (at -6.0325 0.79) (size 0.356 0.356) (layers "B.Cu" "B.Mask" "B.Paste") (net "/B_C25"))
  (pad "C26" smd circle (at -6.667499 0.79) (size 0.356 0.356) (layers "B.Cu" "B.Mask" "B.Paste") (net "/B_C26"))
  (pad "C27" smd circle (at -7.3025 0.79) (size 0.356 0.356) (layers "B.Cu" "B.Mask" "B.Paste") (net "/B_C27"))
  (pad "C28" smd circle (at -7.9375 0.79) (size 0.356 0.356) (layers "B.Cu" "B.Mask" "B.Paste") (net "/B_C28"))
  (pad "C29" smd circle (at -8.572499 0.79) (size 0.356 0.356) (layers "B.Cu" "B.Mask" "B.Paste") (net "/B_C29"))
  (pad "C30" smd circle (at -9.2075 0.79) (size 0.356 0.356) (layers "B.Cu" "B.Mask" "B.Paste") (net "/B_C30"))
  (pad "D01" smd circle (at 9.2075 1.75) (size 0.356 0.356) (layers "B.Cu" "B.Mask" "B.Paste") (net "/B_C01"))
  (pad "D02" smd circle (at 8.5725 1.75) (size 0.356 0.356) (layers "B.Cu" "B.Mask" "B.Paste") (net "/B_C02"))
  (pad "D03" smd circle (at 7.9375 1.75) (size 0.356 0.356) (layers "B.Cu" "B.Mask" "B.Paste") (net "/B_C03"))
  (pad "D04" smd circle (at 7.3025 1.75) (size 0.356 0.356) (layers "B.Cu" "B.Mask" "B.Paste") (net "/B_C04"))
  (pad "D05" smd circle (at 6.6675 1.75) (size 0.356 0.356) (layers "B.Cu" "B.Mask" "B.Paste") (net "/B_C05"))
  (pad "D06" smd circle (at 6.0325 1.75) (size 0.356 0.356) (layers "B.Cu" "B.Mask" "B.Paste") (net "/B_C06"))
  (pad "D07" smd circle (at 5.3975 1.75) (size 0.356 0.356) (layers "B.Cu" "B.Mask" "B.Paste") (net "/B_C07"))
  (pad "D08" smd circle (at 4.7625 1.75) (size 0.356 0.356) (layers "B.Cu" "B.Mask" "B.Paste") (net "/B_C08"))
  (pad "D09" smd circle (at 4.1275 1.75) (size 0.356 0.356) (layers "B.Cu" "B.Mask" "B.Paste") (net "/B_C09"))
  (pad "D10" smd circle (at 3.4925 1.75) (size 0.356 0.356) (layers "B.Cu" "B.Mask" "B.Paste") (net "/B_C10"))
  (pad "D11" smd circle (at 2.8575 1.75) (size 0.356 0.356) (layers "B.Cu" "B.Mask" "B.Paste") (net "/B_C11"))
  (pad "D12" smd circle (at 2.2225 1.75) (size 0.356 0.356) (layers "B.Cu" "B.Mask" "B.Paste") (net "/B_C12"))
  (pad "D13" smd circle (at 1.5875 1.75) (size 0.356 0.356) (layers "B.Cu" "B.Mask" "B.Paste") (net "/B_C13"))
  (pad "D14" smd circle (at 0.9525 1.75) (size 0.356 0.356) (layers "B.Cu" "B.Mask" "B.Paste") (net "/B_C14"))
  (pad "D15" smd circle (at 0.3175 1.75) (size 0.356 0.356) (layers "B.Cu" "B.Mask" "B.Paste") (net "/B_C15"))
  (pad "D16" smd circle (at -0.3175 1.75) (size 0.356 0.356) (layers "B.Cu" "B.Mask" "B.Paste") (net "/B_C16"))
  (pad "D17" smd circle (at -0.9525 1.75) (size 0.356 0.356) (layers "B.Cu" "B.Mask" "B.Paste") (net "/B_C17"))
  (pad "D18" smd circle (at -1.5875 1.75) (size 0.356 0.356) (layers "B.Cu" "B.Mask" "B.Paste") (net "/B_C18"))
  (pad "D19" smd circle (at -2.2225 1.75) (size 0.356 0.356) (layers "B.Cu" "B.Mask" "B.Paste") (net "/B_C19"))
  (pad "D20" smd circle (at -2.8575 1.75) (size 0.356 0.356) (layers "B.Cu" "B.Mask" "B.Paste") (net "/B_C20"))
  (pad "D21" smd circle (at -3.4925 1.75) (size 0.356 0.356) (layers "B.Cu" "B.Mask" "B.Paste") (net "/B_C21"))
  (pad "D22" smd circle (at -4.1275 1.75) (size 0.356 0.356) (layers "B.Cu" "B.Mask" "B.Paste") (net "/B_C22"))
  (pad "D23" smd circle (at -4.762499 1.75) (size 0.356 0.356) (layers "B.Cu" "B.Mask" "B.Paste") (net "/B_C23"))
  (pad "D24" smd circle (at -5.3975 1.75) (size 0.356 0.356) (layers "B.Cu" "B.Mask" "B.Paste") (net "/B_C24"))
  (pad "D25" smd circle (at -6.0325 1.75) (size 0.356 0.356) (layers "B.Cu" "B.Mask" "B.Paste") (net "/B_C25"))
  (pad "D26" smd circle (at -6.667499 1.75) (size 0.356 0.356) (layers "B.Cu" "B.Mask" "B.Paste") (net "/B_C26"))
  (pad "D27" smd circle (at -7.3025 1.75) (size 0.356 0.356) (layers "B.Cu" "B.Mask" "B.Paste") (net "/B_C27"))
  (pad "D28" smd circle (at -7.9375 1.75) (size 0.356 0.356) (layers "B.Cu" "B.Mask" "B.Paste") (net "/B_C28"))
  (pad "D29" smd circle (at -8.572499 1.75) (size 0.356 0.356) (layers "B.Cu" "B.Mask" "B.Paste") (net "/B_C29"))
  (pad "D30" smd circle (at -9.2075 1.75) (size 0.356 0.356) (layers "B.Cu" "B.Mask" "B.Paste") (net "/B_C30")))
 (gr_rect (start 100 100) (end 150 140) (stroke (width 0.1) (type solid)) (fill no) (layer "Edge.Cuts"))
 (segment (start 134.2075 103.25) (end 134.2075 104.21) (width 0.2) (layer "B.Cu") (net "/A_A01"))
 (segment (start 133.5725 103.25) (end 133.5725 104.21) (width 0.2) (layer "B.Cu") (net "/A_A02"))
 (segment (start 132.9375 103.25) (end 132.9375 104.21) (width 0.2) (layer "B.Cu") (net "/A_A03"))
 (segment (start 132.3025 103.25) (end 132.3025 104.21) (width 0.2) (layer "B.Cu") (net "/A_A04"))
 (segment (start 131.6675 103.25) (end 131.6675 104.21) (width 0.2) (layer "B.Cu") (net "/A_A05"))
 (segment (start 131.0325 103.25) (end 131.0325 104.21) (width 0.2) (layer "B.Cu") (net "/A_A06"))
 (segment (start 130.3975 103.25) (end 130.3975 104.21) (width 0.2) (layer "B.Cu") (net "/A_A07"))
 (segment (start 129.7625 103.25) (end 129.7625 104.21) (width 0.2) (layer "B.Cu") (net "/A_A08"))
 (segment (start 129.1275 103.25) (end 129.1275 104.21) (width 0.2) (layer "B.Cu") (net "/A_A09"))
 (segment (start 128.4925 103.25) (end 128.4925 104.21) (width 0.2) (layer "B.Cu") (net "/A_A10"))
 (segment (start 127.8575 103.25) (end 127.8575 104.21) (width 0.2) (layer "B.Cu") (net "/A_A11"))
 (segment (start 127.2225 103.25) (end 127.2225 104.21) (width 0.2) (layer "B.Cu") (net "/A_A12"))
 (segment (start 126.5875 103.25) (end 126.5875 104.21) (width 0.2) (layer "B.Cu") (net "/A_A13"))
 (segment (start 125.9525 103.25) (end 125.9525 104.21) (width 0.2) (layer "B.Cu") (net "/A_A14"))
 (segment (start 125.3175 103.25) (end 125.3175 104.21) (width 0.2) (layer "B.Cu") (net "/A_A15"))
 (segment (start 124.6825 103.25) (end 124.6825 104.21) (width 0.2) (layer "B.Cu") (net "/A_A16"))
 (segment (start 124.0475 103.25) (end 124.0475 104.21) (width 0.2) (layer "B.Cu") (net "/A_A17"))
 (segment (start 123.4125 103.25) (end 123.4125 104.21) (width 0.2) (layer "B.Cu") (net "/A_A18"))
 (segment (start 122.7775 103.25) (end 122.7775 104.21) (width 0.2) (layer "B.Cu") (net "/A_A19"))
 (segment (start 122.1425 103.25) (end 122.1425 104.21) (width 0.2) (layer "B.Cu") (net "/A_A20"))
 (segment (start 121.5075 103.25) (end 121.5075 104.21) (width 0.2) (layer "B.Cu") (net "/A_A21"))
 (segment (start 120.8725 103.25) (end 120.8725 104.21) (width 0.2) (layer "B.Cu") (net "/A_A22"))
 (segment (start 120.237501 103.25) (end 120.237501 104.21) (width 0.2) (layer "B.Cu") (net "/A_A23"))
 (segment (start 119.6025 103.25) (end 119.6025 104.21) (width 0.2) (layer "B.Cu") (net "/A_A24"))
 (segment (start 118.9675 103.25) (end 118.9675 104.21) (width 0.2) (layer "B.Cu") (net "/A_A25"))
 (segment (start 118.332501 103.25) (end 118.332501 104.21) (width 0.2) (layer "B.Cu") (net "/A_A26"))
 (segment (start 117.6975 103.25) (end 117.6975 104.21) (width 0.2) (layer "B.Cu") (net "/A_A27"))
 (segment (start 117.0625 103.25) (end 117.0625 104.21) (width 0.2) (layer "B.Cu") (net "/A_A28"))
 (segment (start 116.427501 103.25) (end 116.427501 104.21) (width 0.2) (layer "B.Cu") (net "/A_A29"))
 (segment (start 115.7925 103.25) (end 115.7925 104.21) (width 0.2) (layer "B.Cu") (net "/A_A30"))
 (segment (start 134.2075 105.79) (end 134.2075 106.75) (width 0.2) (layer "B.Cu") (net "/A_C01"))
 (segment (start 133.5725 105.79) (end 133.5725 106.75) (width 0.2) (layer "B.Cu") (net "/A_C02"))
 (segment (start 132.9375 105.79) (end 132.9375 106.75) (width 0.2) (layer "B.Cu") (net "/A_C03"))
 (segment (start 132.3025 105.79) (end 132.3025 106.75) (width 0.2) (layer "B.Cu") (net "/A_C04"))
 (segment (start 131.6675 105.79) (end 131.6675 106.75) (width 0.2) (layer "B.Cu") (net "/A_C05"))
 (segment (start 131.0325 105.79) (end 131.0325 106.75) (width 0.2) (layer "B.Cu") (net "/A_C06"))
 (segment (start 130.3975 105.79) (end 130.3975 106.75) (width 0.2) (layer "B.Cu") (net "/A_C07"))
 (segment (start 129.7625 105.79) (end 129.7625 106.75) (width 0.2) (layer "B.Cu") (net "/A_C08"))
 (segment (start 129.1275 105.79) (end 129.1275 106.75) (width 0.2) (layer "B.Cu") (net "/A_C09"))
 (segment (start 128.4925 105.79) (end 128.4925 106.75) (width 0.2) (layer "B.Cu") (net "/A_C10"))
 (segment (start 127.8575 105.79) (end 127.8575 106.75) (width 0.2) (layer "B.Cu") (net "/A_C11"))
 (segment (start 127.2225 105.79) (end 127.2225 106.75) (width 0.2) (layer "B.Cu") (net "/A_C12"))
 (segment (start 126.5875 105.79) (end 126.5875 106.75) (width 0.2) (layer "B.Cu") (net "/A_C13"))
 (segment (start 125.9525 105.79) (end 125.9525 106.75) (width 0.2) (layer "B.Cu") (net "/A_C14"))
 (segment (start 125.3175 105.79) (end 125.3175 106.75) (width 0.2) (layer "B.Cu") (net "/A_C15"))
 (segment (start 124.6825 105.79) (end 124.6825 106.75) (width 0.2) (layer "B.Cu") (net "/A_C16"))
 (segment (start 124.0475 105.79) (end 124.0475 106.75) (width 0.2) (layer "B.Cu") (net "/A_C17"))
 (segment (start 123.4125 105.79) (end 123.4125 106.75) (width 0.2) (layer "B.Cu") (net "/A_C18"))
 (segment (start 122.7775 105.79) (end 122.7775 106.75) (width 0.2) (layer "B.Cu") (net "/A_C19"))
 (segment (start 122.1425 105.79) (end 122.1425 106.75) (width 0.2) (layer "B.Cu") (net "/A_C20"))
 (segment (start 121.5075 105.79) (end 121.5075 106.75) (width 0.2) (layer "B.Cu") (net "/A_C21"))
 (segment (start 120.8725 105.79) (end 120.8725 106.75) (width 0.2) (layer "B.Cu") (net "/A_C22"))
 (segment (start 120.237501 105.79) (end 120.237501 106.75) (width 0.2) (layer "B.Cu") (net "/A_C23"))
 (segment (start 119.6025 105.79) (end 119.6025 106.75) (width 0.2) (layer "B.Cu") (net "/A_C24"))
 (segment (start 118.9675 105.79) (end 118.9675 106.75) (width 0.2) (layer "B.Cu") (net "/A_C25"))
 (segment (start 118.332501 105.79) (end 118.332501 106.75) (width 0.2) (layer "B.Cu") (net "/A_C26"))
 (segment (start 117.6975 105.79) (end 117.6975 106.75) (width 0.2) (layer "B.Cu") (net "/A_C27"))
 (segment (start 117.0625 105.79) (end 117.0625 106.75) (width 0.2) (layer "B.Cu") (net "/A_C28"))
 (segment (start 116.427501 105.79) (end 116.427501 106.75) (width 0.2) (layer "B.Cu") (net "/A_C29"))
 (segment (start 115.7925 105.79) (end 115.7925 106.75) (width 0.2) (layer "B.Cu") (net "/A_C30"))
 (segment (start 134.2075 133.25) (end 134.2075 134.21) (width 0.2) (layer "B.Cu") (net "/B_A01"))
 (segment (start 133.5725 133.25) (end 133.5725 134.21) (width 0.2) (layer "B.Cu") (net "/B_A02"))
 (segment (start 132.9375 133.25) (end 132.9375 134.21) (width 0.2) (layer "B.Cu") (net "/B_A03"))
 (segment (start 132.3025 133.25) (end 132.3025 134.21) (width 0.2) (layer "B.Cu") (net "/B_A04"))
 (segment (start 131.6675 133.25) (end 131.6675 134.21) (width 0.2) (layer "B.Cu") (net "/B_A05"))
 (segment (start 131.0325 133.25) (end 131.0325 134.21) (width 0.2) (layer "B.Cu") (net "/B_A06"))
 (segment (start 130.3975 133.25) (end 130.3975 134.21) (width 0.2) (layer "B.Cu") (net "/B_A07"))
 (segment (start 129.7625 133.25) (end 129.7625 134.21) (width 0.2) (layer "B.Cu") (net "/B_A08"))
 (segment (start 129.1275 133.25) (end 129.1275 134.21) (width 0.2) (layer "B.Cu") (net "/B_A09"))
 (segment (start 128.4925 133.25) (end 128.4925 134.21) (width 0.2) (layer "B.Cu") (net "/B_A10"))
 (segment (start 127.8575 133.25) (end 127.8575 134.21) (width 0.2) (layer "B.Cu") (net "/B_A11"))
 (segment (start 127.2225 133.25) (end 127.2225 134.21) (width 0.2) (layer "B.Cu") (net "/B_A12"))
 (segment (start 126.5875 133.25) (end 126.5875 134.21) (width 0.2) (layer "B.Cu") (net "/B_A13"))
 (segment (start 125.9525 133.25) (end 125.9525 134.21) (width 0.2) (layer "B.Cu") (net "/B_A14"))
 (segment (start 125.3175 133.25) (end 125.3175 134.21) (width 0.2) (layer "B.Cu") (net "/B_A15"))
 (segment (start 124.6825 133.25) (end 124.6825 134.21) (width 0.2) (layer "B.Cu") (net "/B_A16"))
 (segment (start 124.0475 133.25) (end 124.0475 134.21) (width 0.2) (layer "B.Cu") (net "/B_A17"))
 (segment (start 123.4125 133.25) (end 123.4125 134.21) (width 0.2) (layer "B.Cu") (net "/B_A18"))
 (segment (start 122.7775 133.25) (end 122.7775 134.21) (width 0.2) (layer "B.Cu") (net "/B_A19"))
 (segment (start 122.1425 133.25) (end 122.1425 134.21) (width 0.2) (layer "B.Cu") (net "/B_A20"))
 (segment (start 121.5075 133.25) (end 121.5075 134.21) (width 0.2) (layer "B.Cu") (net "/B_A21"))
 (segment (start 120.8725 133.25) (end 120.8725 134.21) (width 0.2) (layer "B.Cu") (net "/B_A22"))
 (segment (start 120.237501 133.25) (end 120.237501 134.21) (width 0.2) (layer "B.Cu") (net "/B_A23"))
 (segment (start 119.6025 133.25) (end 119.6025 134.21) (width 0.2) (layer "B.Cu") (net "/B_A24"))
 (segment (start 118.9675 133.25) (end 118.9675 134.21) (width 0.2) (layer "B.Cu") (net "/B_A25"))
 (segment (start 118.332501 133.25) (end 118.332501 134.21) (width 0.2) (layer "B.Cu") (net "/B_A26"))
 (segment (start 117.6975 133.25) (end 117.6975 134.21) (width 0.2) (layer "B.Cu") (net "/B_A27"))
 (segment (start 117.0625 133.25) (end 117.0625 134.21) (width 0.2) (layer "B.Cu") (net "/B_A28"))
 (segment (start 116.427501 133.25) (end 116.427501 134.21) (width 0.2) (layer "B.Cu") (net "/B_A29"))
 (segment (start 115.7925 133.25) (end 115.7925 134.21) (width 0.2) (layer "B.Cu") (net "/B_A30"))
 (segment (start 134.2075 135.79) (end 134.2075 136.75) (width 0.2) (layer "B.Cu") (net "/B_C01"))
 (segment (start 133.5725 135.79) (end 133.5725 136.75) (width 0.2) (layer "B.Cu") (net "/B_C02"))
 (segment (start 132.9375 135.79) (end 132.9375 136.75) (width 0.2) (layer "B.Cu") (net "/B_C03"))
 (segment (start 132.3025 135.79) (end 132.3025 136.75) (width 0.2) (layer "B.Cu") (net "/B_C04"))
 (segment (start 131.6675 135.79) (end 131.6675 136.75) (width 0.2) (layer "B.Cu") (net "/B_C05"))
 (segment (start 131.0325 135.79) (end 131.0325 136.75) (width 0.2) (layer "B.Cu") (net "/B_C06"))
 (segment (start 130.3975 135.79) (end 130.3975 136.75) (width 0.2) (layer "B.Cu") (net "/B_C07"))
 (segment (start 129.7625 135.79) (end 129.7625 136.75) (width 0.2) (layer "B.Cu") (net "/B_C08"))
 (segment (start 129.1275 135.79) (end 129.1275 136.75) (width 0.2) (layer "B.Cu") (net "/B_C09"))
 (segment (start 128.4925 135.79) (end 128.4925 136.75) (width 0.2) (layer "B.Cu") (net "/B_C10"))
 (segment (start 127.8575 135.79) (end 127.8575 136.75) (width 0.2) (layer "B.Cu") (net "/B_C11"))
 (segment (start 127.2225 135.79) (end 127.2225 136.75) (width 0.2) (layer "B.Cu") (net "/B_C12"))
 (segment (start 126.5875 135.79) (end 126.5875 136.75) (width 0.2) (layer "B.Cu") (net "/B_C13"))
 (segment (start 125.9525 135.79) (end 125.9525 136.75) (width 0.2) (layer "B.Cu") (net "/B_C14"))
 (segment (start 125.3175 135.79) (end 125.3175 136.75) (width 0.2) (layer "B.Cu") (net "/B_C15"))
 (segment (start 124.6825 135.79) (end 124.6825 136.75) (width 0.2) (layer "B.Cu") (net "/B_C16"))
 (segment (start 124.0475 135.79) (end 124.0475 136.75) (width 0.2) (layer "B.Cu") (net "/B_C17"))
 (segment (start 123.4125 135.79) (end 123.4125 136.75) (width 0.2) (layer "B.Cu") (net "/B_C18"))
 (segment (start 122.7775 135.79) (end 122.7775 136.75) (width 0.2) (layer "B.Cu") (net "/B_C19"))
 (segment (start 122.1425 135.79) (end 122.1425 136.75) (width 0.2) (layer "B.Cu") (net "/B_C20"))
 (segment (start 121.5075 135.79) (end 121.5075 136.75) (width 0.2) (layer "B.Cu") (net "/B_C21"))
 (segment (start 120.8725 135.79) (end 120.8725 136.75) (width 0.2) (layer "B.Cu") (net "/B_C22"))
 (segment (start 120.237501 135.79) (end 120.237501 136.75) (width 0.2) (layer "B.Cu") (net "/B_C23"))
 (segment (start 119.6025 135.79) (end 119.6025 136.75) (width 0.2) (layer "B.Cu") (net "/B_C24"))
 (segment (start 118.9675 135.79) (end 118.9675 136.75) (width 0.2) (layer "B.Cu") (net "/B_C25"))
 (segment (start 118.332501 135.79) (end 118.332501 136.75) (width 0.2) (layer "B.Cu") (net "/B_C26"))
 (segment (start 117.6975 135.79) (end 117.6975 136.75) (width 0.2) (layer "B.Cu") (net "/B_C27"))
 (segment (start 117.0625 135.79) (end 117.0625 136.75) (width 0.2) (layer "B.Cu") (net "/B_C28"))
 (segment (start 116.427501 135.79) (end 116.427501 136.75) (width 0.2) (layer "B.Cu") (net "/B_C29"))
 (segment (start 115.7925 135.79) (end 115.7925 136.75) (width 0.2) (layer "B.Cu") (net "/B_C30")))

